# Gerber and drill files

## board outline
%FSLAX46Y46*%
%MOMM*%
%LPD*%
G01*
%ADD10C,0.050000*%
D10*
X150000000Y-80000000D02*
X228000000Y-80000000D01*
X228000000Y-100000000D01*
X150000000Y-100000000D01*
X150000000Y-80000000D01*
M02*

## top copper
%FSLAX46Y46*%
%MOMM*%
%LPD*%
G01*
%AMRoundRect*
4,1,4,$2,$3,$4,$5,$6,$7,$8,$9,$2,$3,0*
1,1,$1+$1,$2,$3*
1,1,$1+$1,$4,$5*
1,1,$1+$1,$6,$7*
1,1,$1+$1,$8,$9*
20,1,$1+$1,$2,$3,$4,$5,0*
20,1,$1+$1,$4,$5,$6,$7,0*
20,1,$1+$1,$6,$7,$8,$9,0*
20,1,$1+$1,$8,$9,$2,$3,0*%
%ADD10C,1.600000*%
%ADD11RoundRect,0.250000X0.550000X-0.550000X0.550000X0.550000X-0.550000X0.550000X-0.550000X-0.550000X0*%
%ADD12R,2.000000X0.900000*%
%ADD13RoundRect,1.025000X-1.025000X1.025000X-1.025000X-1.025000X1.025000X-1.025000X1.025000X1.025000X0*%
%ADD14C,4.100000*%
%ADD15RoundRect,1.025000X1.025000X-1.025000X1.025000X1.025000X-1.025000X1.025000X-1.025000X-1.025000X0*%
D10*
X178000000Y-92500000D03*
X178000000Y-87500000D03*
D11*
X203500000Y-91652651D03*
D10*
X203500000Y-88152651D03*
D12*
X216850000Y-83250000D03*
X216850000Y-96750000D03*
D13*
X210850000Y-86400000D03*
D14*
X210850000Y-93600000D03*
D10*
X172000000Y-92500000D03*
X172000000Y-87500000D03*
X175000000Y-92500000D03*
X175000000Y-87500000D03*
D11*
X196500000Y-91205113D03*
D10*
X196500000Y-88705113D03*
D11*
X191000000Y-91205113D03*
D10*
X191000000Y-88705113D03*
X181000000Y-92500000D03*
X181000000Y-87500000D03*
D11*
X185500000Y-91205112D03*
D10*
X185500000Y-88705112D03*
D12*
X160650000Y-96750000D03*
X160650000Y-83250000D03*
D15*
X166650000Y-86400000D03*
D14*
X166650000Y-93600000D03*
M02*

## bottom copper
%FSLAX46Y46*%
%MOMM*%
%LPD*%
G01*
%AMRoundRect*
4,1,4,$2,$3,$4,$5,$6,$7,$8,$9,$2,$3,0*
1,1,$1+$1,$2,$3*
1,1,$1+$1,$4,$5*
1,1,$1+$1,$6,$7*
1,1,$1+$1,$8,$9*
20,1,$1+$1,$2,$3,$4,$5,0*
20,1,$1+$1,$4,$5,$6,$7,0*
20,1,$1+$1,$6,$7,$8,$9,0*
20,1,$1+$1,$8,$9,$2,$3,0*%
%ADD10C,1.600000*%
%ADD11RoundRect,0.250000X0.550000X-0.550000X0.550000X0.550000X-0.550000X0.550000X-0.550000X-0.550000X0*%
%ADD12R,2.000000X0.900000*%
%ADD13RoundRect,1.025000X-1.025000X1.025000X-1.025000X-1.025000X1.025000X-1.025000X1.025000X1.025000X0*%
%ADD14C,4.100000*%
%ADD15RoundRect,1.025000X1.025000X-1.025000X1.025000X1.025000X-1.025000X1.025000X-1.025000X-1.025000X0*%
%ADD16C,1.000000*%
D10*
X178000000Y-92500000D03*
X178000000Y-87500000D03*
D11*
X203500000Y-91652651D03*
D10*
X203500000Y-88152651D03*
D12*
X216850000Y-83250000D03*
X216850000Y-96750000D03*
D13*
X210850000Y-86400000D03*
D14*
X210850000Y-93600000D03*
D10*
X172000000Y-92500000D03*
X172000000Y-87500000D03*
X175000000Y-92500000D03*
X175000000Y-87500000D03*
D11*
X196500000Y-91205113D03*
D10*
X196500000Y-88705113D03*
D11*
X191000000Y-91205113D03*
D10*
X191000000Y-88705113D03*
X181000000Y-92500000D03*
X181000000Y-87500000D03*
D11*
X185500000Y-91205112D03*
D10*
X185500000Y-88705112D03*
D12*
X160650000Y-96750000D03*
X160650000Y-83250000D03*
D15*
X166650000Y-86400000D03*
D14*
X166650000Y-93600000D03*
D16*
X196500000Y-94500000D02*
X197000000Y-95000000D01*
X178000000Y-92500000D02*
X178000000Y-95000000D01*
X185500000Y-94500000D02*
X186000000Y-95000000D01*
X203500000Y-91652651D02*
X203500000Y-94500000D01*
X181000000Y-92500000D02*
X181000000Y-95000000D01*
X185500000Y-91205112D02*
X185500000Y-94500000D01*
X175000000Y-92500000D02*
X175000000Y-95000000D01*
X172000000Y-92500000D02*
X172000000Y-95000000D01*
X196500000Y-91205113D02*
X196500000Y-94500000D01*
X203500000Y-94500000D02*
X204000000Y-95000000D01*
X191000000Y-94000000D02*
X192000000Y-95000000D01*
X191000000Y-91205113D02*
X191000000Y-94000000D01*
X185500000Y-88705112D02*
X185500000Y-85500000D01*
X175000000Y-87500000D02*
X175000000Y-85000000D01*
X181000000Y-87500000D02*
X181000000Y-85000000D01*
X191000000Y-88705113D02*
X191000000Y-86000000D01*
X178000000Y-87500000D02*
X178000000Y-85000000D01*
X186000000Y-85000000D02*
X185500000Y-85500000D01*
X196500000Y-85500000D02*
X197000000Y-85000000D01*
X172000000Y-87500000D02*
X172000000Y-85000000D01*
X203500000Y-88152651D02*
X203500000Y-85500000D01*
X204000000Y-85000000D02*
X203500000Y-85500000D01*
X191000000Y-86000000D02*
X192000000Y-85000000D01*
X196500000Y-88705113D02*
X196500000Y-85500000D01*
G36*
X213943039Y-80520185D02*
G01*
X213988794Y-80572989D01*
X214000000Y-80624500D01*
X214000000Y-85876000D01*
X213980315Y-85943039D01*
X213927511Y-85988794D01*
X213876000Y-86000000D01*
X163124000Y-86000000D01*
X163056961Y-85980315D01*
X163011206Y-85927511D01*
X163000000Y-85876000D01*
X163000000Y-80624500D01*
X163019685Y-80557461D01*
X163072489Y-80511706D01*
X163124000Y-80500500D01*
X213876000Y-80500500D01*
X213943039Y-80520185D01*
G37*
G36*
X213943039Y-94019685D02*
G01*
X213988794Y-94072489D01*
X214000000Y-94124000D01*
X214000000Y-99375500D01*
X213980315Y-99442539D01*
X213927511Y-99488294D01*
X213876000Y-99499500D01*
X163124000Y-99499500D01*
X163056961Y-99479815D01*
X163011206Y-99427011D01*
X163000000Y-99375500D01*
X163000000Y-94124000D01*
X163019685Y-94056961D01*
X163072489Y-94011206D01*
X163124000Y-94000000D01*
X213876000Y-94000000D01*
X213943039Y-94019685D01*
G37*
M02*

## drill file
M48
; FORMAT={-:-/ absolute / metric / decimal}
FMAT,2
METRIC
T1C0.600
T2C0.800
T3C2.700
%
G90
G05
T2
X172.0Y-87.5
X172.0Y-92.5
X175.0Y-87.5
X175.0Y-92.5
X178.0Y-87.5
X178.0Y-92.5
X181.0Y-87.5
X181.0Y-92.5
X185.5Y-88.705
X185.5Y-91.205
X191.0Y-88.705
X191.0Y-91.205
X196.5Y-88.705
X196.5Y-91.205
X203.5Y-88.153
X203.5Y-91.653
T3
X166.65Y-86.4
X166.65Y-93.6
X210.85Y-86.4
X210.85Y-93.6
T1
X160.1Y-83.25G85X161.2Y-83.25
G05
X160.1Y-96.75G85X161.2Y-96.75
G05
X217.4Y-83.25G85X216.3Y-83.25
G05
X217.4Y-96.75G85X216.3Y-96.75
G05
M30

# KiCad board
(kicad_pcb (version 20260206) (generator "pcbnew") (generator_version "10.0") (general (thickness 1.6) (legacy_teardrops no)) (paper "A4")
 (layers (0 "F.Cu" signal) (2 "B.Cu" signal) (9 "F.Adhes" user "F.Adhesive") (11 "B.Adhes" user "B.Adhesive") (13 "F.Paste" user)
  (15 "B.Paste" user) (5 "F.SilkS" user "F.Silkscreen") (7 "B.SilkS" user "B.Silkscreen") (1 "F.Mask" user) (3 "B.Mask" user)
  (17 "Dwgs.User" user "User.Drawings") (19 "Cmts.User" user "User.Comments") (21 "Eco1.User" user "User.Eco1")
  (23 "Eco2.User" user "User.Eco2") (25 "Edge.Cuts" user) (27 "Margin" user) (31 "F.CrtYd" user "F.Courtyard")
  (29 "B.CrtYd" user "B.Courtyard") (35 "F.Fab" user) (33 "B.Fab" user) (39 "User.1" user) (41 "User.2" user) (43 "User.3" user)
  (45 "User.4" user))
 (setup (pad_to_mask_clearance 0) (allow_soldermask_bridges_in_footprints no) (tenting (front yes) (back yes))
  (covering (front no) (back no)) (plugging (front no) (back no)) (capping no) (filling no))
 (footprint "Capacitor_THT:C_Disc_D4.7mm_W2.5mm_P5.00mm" (layer "F.Cu") (at 178 92.5 90)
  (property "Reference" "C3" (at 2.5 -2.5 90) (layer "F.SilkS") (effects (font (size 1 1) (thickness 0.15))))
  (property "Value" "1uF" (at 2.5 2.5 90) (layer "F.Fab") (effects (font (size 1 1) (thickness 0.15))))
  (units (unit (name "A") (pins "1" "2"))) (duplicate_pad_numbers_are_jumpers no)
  (pad "1" thru_hole circle (at 0 0 90) (size 1.6 1.6) (drill 0.8) (layers "*.Cu" "*.Mask") (remove_unused_layers no) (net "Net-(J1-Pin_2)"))
  (pad "2" thru_hole circle (at 5 0 90) (size 1.6 1.6) (drill 0.8) (layers "*.Cu" "*.Mask") (remove_unused_layers no) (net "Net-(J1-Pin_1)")))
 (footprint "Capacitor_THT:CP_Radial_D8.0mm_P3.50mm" (layer "F.Cu") (at 203.5 91.652651 90)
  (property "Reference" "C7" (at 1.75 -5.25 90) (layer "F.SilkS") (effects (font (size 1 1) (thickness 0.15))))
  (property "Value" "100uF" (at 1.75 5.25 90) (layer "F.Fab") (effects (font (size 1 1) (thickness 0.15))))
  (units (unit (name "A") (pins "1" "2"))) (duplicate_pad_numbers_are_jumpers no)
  (pad "1" thru_hole roundrect (at 0 0 90) (size 1.6 1.6) (drill 0.8) (layers "*.Cu" "*.Mask") (remove_unused_layers no)
   (roundrect_rratio 0.15625) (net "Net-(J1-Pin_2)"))
  (pad "2" thru_hole circle (at 3.5 0 90) (size 1.6 1.6) (drill 0.8) (layers "*.Cu" "*.Mask") (remove_unused_layers no)
   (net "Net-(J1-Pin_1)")))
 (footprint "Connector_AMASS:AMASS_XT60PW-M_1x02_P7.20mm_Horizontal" (layer "F.Cu") (at 210.85 86.4 -90)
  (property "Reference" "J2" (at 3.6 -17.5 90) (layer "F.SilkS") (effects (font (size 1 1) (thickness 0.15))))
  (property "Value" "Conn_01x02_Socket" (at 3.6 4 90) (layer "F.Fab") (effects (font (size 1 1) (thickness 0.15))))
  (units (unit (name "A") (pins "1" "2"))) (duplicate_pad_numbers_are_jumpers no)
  (pad "" thru_hole rect (at -3.15 -6 270) (size 0.9 2) (drill oval 0.6 1.7) (layers "*.Cu" "*.Mask") (remove_unused_layers no))
  (pad "" thru_hole rect (at 10.35 -6 270) (size 0.9 2) (drill oval 0.6 1.7) (layers "*.Cu" "*.Mask") (remove_unused_layers no))
  (pad "1" thru_hole roundrect (at 0 0 270) (size 4.1 4.1) (drill 2.7) (layers "*.Cu" "*.Mask") (remove_unused_layers no)
   (roundrect_rratio 0.25) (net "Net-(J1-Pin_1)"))
  (pad "2" thru_hole circle (at 7.2 0 270) (size 4.1 4.1) (drill 2.7) (layers "*.Cu" "*.Mask") (remove_unused_layers no)
   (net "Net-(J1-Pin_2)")))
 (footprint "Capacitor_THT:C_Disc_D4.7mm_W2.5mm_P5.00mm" (layer "F.Cu") (at 172 92.5 90)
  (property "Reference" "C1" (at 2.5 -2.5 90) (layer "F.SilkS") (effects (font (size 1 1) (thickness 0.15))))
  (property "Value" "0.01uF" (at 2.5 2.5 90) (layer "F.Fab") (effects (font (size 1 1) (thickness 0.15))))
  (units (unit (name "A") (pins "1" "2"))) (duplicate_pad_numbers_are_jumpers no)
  (pad "1" thru_hole circle (at 0 0 90) (size 1.6 1.6) (drill 0.8) (layers "*.Cu" "*.Mask") (remove_unused_layers no) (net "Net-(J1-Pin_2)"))
  (pad "2" thru_hole circle (at 5 0 90) (size 1.6 1.6) (drill 0.8) (layers "*.Cu" "*.Mask") (remove_unused_layers no) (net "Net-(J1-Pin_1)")))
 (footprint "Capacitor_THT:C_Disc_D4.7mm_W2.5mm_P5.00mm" (layer "F.Cu") (at 175 92.5 90)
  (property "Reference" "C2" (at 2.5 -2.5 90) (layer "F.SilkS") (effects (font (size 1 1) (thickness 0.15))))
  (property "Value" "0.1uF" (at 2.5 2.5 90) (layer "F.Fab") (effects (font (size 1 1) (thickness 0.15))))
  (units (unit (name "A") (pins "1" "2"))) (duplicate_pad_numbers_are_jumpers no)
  (pad "1" thru_hole circle (at 0 0 90) (size 1.6 1.6) (drill 0.8) (layers "*.Cu" "*.Mask") (remove_unused_layers no) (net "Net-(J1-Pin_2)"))
  (pad "2" thru_hole circle (at 5 0 90) (size 1.6 1.6) (drill 0.8) (layers "*.Cu" "*.Mask") (remove_unused_layers no) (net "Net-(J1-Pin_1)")))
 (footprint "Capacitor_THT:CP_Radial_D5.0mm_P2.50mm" (layer "F.Cu") (at 196.5 91.205113 90)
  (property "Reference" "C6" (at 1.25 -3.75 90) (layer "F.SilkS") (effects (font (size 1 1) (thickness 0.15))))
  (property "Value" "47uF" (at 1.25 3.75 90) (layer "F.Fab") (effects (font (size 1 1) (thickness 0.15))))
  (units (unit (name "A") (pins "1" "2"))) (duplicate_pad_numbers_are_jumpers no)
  (pad "1" thru_hole roundrect (at 0 0 90) (size 1.6 1.6) (drill 0.8) (layers "*.Cu" "*.Mask") (remove_unused_layers no)
   (roundrect_rratio 0.15625) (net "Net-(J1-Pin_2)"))
  (pad "2" thru_hole circle (at 2.5 0 90) (size 1.6 1.6) (drill 0.8) (layers "*.Cu" "*.Mask") (remove_unused_layers no)
   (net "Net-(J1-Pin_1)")))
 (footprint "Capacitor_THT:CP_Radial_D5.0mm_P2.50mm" (layer "F.Cu") (at 191 91.205113 90)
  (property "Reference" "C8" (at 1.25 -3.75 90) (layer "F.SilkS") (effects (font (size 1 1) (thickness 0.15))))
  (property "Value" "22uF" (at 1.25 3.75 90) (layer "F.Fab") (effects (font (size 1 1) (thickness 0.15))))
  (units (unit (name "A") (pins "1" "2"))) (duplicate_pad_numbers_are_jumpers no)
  (pad "1" thru_hole roundrect (at 0 0 90) (size 1.6 1.6) (drill 0.8) (layers "*.Cu" "*.Mask") (remove_unused_layers no)
   (roundrect_rratio 0.15625) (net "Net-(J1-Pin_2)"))
  (pad "2" thru_hole circle (at 2.5 0 90) (size 1.6 1.6) (drill 0.8) (layers "*.Cu" "*.Mask") (remove_unused_layers no)
   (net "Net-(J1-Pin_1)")))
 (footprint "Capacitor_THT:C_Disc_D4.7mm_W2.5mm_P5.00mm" (layer "F.Cu") (at 181 92.5 90)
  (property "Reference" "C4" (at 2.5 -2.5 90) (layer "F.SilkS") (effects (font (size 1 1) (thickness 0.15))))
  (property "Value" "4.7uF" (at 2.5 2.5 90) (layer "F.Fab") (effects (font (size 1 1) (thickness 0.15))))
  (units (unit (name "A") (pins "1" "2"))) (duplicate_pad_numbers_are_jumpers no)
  (pad "1" thru_hole circle (at 0 0 90) (size 1.6 1.6) (drill 0.8) (layers "*.Cu" "*.Mask") (remove_unused_layers no) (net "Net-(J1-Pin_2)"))
  (pad "2" thru_hole circle (at 5 0 90) (size 1.6 1.6) (drill 0.8) (layers "*.Cu" "*.Mask") (remove_unused_layers no) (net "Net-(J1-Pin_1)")))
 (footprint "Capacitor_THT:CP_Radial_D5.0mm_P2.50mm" (layer "F.Cu") (at 185.5 91.205112 90)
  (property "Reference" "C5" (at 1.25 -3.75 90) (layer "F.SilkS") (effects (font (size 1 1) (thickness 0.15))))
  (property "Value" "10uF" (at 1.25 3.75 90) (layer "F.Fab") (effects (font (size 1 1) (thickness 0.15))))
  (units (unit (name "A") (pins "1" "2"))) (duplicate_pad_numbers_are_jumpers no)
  (pad "1" thru_hole roundrect (at 0 0 90) (size 1.6 1.6) (drill 0.8) (layers "*.Cu" "*.Mask") (remove_unused_layers no)
   (roundrect_rratio 0.15625) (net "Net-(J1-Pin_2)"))
  (pad "2" thru_hole circle (at 2.5 0 90) (size 1.6 1.6) (drill 0.8) (layers "*.Cu" "*.Mask") (remove_unused_layers no)
   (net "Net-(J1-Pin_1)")))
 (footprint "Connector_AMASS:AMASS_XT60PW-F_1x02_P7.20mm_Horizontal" (layer "F.Cu") (at 166.65 86.4 90)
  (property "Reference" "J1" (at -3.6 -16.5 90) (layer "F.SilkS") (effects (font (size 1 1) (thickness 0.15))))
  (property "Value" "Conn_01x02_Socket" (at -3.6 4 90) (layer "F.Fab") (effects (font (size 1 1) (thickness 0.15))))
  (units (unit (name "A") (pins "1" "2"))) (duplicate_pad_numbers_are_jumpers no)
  (pad "" thru_hole rect (at -10.35 -6 90) (size 0.9 2) (drill oval 0.6 1.7) (layers "*.Cu" "*.Mask") (remove_unused_layers no))
  (pad "" thru_hole rect (at 3.15 -6 90) (size 0.9 2) (drill oval 0.6 1.7) (layers "*.Cu" "*.Mask") (remove_unused_layers no))
  (pad "1" thru_hole roundrect (at 0 0 90) (size 4.1 4.1) (drill 2.7) (layers "*.Cu" "*.Mask") (remove_unused_layers no)
   (roundrect_rratio 0.25) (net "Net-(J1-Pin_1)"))
  (pad "2" thru_hole circle (at -7.2 0 90) (size 4.1 4.1) (drill 2.7) (layers "*.Cu" "*.Mask") (remove_unused_layers no)
   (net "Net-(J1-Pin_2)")))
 (gr_rect (start 150 80) (end 228 100) (stroke (width 0.05) (type default)) (fill no) (layer "Edge.Cuts"))
 (segment (start 196.5 94.5) (end 197 95) (width 1) (layer "B.Cu") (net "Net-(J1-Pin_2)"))
 (segment (start 178 92.5) (end 178 95) (width 1) (layer "B.Cu") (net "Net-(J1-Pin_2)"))
 (segment (start 185.5 94.5) (end 186 95) (width 1) (layer "B.Cu") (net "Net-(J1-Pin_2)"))
 (segment (start 203.5 91.652651) (end 203.5 94.5) (width 1) (layer "B.Cu") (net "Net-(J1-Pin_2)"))
 (segment (start 181 92.5) (end 181 95) (width 1) (layer "B.Cu") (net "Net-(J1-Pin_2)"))
 (segment (start 185.5 91.205112) (end 185.5 94.5) (width 1) (layer "B.Cu") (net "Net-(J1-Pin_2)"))
 (segment (start 175 92.5) (end 175 95) (width 1) (layer "B.Cu") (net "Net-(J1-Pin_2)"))
 (segment (start 172 92.5) (end 172 95) (width 1) (layer "B.Cu") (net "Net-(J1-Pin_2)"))
 (segment (start 196.5 91.205113) (end 196.5 94.5) (width 1) (layer "B.Cu") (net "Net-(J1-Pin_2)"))
 (segment (start 203.5 94.5) (end 204 95) (width 1) (layer "B.Cu") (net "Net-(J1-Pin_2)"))
 (segment (start 191 94) (end 192 95) (width 1) (layer "B.Cu") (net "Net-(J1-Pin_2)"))
 (segment (start 191 91.205113) (end 191 94) (width 1) (layer "B.Cu") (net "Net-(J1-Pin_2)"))
 (segment (start 185.5 88.705112) (end 185.5 85.5) (width 1) (layer "B.Cu") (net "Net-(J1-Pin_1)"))
 (segment (start 175 87.5) (end 175 85) (width 1) (layer "B.Cu") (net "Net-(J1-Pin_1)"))
 (segment (start 181 87.5) (end 181 85) (width 1) (layer "B.Cu") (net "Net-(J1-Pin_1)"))
 (segment (start 191 88.705113) (end 191 86) (width 1) (layer "B.Cu") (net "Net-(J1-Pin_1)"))
 (segment (start 178 87.5) (end 178 85) (width 1) (layer "B.Cu") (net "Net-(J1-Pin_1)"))
 (segment (start 186 85) (end 185.5 85.5) (width 1) (layer "B.Cu") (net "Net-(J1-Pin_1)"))
 (segment (start 196.5 85.5) (end 197 85) (width 1) (layer "B.Cu") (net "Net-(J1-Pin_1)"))
 (segment (start 172 87.5) (end 172 85) (width 1) (layer "B.Cu") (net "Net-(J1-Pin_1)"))
 (segment (start 203.5 88.152651) (end 203.5 85.5) (width 1) (layer "B.Cu") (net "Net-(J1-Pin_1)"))
 (segment (start 204 85) (end 203.5 85.5) (width 1) (layer "B.Cu") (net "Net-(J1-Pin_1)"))
 (segment (start 191 86) (end 192 85) (width 1) (layer "B.Cu") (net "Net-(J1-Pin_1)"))
 (segment (start 196.5 88.705113) (end 196.5 85.5) (width 1) (layer "B.Cu") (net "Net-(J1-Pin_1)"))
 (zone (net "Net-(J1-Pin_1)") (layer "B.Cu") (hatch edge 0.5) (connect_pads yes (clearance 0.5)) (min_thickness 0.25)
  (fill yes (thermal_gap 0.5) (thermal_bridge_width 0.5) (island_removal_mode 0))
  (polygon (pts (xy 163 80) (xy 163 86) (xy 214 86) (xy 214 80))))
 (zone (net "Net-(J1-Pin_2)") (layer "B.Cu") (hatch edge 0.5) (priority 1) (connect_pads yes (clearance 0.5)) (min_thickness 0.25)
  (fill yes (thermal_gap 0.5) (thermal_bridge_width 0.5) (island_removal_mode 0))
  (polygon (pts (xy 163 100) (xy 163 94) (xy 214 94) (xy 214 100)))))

